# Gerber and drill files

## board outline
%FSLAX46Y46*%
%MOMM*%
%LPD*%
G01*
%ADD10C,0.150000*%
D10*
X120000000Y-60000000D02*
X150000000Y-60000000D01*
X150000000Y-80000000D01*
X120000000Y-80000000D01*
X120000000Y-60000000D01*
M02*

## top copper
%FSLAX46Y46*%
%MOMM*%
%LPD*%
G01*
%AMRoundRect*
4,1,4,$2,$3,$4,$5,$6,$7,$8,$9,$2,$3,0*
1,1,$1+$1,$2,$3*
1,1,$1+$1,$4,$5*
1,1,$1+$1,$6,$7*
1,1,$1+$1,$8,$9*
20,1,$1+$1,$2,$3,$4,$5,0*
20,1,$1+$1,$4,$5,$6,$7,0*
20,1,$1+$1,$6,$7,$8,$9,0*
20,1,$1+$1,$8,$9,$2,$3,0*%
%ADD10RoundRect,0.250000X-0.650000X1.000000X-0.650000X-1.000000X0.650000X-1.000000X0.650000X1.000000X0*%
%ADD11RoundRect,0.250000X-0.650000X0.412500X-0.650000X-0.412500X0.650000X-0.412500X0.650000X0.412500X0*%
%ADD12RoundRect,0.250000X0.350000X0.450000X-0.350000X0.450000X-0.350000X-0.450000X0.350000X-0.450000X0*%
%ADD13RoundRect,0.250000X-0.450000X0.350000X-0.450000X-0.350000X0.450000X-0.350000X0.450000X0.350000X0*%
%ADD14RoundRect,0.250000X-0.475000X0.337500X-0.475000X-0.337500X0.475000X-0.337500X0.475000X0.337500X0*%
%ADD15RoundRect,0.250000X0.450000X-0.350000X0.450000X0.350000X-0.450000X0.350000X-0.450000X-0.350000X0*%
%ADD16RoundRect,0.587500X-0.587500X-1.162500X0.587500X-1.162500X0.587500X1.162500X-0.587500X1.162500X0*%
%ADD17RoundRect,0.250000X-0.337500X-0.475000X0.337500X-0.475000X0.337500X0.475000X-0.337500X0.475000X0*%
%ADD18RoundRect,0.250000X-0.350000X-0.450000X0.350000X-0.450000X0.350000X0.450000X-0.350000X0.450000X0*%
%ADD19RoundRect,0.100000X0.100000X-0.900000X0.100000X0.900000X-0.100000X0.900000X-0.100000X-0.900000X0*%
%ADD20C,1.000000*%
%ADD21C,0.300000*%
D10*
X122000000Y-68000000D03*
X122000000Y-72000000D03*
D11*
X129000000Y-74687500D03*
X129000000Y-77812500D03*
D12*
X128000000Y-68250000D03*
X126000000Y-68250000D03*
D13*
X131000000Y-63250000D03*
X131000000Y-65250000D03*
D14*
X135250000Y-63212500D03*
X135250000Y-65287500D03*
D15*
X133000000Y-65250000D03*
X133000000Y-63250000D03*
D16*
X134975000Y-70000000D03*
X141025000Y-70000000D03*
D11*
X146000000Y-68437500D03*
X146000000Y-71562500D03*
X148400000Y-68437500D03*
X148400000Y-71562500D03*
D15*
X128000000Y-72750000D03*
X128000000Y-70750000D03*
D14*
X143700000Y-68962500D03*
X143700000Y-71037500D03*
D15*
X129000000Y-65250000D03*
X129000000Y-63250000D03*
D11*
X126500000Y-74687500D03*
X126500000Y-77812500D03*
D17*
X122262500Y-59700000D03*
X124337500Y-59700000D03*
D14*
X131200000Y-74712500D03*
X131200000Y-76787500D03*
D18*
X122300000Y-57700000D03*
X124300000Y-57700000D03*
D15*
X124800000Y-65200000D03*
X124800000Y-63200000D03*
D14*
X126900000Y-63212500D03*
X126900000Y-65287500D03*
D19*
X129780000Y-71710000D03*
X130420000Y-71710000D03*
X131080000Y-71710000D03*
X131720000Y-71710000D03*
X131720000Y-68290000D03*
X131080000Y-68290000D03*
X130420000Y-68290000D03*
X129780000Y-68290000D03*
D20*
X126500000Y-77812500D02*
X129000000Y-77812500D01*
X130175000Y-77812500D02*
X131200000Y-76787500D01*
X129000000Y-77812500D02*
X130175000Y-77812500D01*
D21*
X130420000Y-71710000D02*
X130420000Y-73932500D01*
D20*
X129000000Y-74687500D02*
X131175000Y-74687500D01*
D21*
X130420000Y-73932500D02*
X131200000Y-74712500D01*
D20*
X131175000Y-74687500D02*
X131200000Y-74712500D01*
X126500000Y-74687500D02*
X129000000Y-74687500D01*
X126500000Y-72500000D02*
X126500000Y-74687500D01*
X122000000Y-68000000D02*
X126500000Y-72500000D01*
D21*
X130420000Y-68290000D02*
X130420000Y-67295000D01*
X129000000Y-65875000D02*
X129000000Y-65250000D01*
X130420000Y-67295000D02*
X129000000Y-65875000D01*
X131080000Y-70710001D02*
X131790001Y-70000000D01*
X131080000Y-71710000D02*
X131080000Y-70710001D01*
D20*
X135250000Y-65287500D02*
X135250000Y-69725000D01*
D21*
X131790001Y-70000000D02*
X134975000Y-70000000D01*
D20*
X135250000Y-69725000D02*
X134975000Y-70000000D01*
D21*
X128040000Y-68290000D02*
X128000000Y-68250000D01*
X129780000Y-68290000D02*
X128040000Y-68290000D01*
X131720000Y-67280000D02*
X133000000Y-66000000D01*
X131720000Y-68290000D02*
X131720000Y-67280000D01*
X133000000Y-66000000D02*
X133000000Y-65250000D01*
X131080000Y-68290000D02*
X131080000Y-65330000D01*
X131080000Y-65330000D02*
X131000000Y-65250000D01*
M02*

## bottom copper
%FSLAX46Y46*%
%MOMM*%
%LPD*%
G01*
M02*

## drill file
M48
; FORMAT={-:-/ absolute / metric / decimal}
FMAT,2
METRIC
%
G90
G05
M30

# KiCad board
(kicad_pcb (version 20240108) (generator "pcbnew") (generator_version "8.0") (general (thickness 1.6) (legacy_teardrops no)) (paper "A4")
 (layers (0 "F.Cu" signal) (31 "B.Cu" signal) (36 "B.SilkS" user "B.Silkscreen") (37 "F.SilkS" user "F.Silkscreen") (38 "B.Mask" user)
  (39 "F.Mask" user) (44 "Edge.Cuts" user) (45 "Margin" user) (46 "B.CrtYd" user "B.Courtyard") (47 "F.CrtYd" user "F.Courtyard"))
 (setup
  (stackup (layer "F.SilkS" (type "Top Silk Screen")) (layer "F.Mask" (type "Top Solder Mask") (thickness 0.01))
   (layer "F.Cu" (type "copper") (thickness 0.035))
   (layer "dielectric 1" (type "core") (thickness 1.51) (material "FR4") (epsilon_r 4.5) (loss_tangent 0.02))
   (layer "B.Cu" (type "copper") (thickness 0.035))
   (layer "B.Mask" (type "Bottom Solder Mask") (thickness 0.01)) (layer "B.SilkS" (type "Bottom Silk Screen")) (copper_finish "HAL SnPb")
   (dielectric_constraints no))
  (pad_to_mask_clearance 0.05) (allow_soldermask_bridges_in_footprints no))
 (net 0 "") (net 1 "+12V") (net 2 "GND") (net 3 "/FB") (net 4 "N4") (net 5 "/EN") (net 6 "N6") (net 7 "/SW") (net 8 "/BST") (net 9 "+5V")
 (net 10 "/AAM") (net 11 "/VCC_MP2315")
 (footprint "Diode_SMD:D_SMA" (layer "F.Cu") (at 122 70 -90)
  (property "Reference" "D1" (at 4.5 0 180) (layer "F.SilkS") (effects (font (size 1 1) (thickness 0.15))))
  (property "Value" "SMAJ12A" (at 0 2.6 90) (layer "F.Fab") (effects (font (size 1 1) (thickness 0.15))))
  (pad "1" smd roundrect (at -2 0 270) (size 2.5 1.8) (layers "F.Cu" "F.Paste" "F.Mask") (roundrect_rratio 0.1388888889) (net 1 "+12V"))
  (pad "2" smd roundrect (at 2 0 270) (size 2.5 1.8) (layers "F.Cu" "F.Paste" "F.Mask") (roundrect_rratio 0.1388888889) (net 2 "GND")))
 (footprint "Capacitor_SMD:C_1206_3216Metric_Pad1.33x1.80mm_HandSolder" (layer "F.Cu") (at 129 76.25 -90)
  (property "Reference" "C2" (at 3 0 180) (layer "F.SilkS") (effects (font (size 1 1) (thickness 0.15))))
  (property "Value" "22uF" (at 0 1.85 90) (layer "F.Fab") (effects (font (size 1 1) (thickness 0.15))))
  (pad "1" smd roundrect (at -1.5625 0 270) (size 1.325 1.8) (layers "F.Cu" "F.Paste" "F.Mask") (roundrect_rratio 0.188679) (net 1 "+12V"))
  (pad "2" smd roundrect (at 1.5625 0 270) (size 1.325 1.8) (layers "F.Cu" "F.Paste" "F.Mask") (roundrect_rratio 0.188679) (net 2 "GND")))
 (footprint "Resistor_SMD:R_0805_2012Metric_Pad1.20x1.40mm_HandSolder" (layer "F.Cu") (at 127 68.25 180)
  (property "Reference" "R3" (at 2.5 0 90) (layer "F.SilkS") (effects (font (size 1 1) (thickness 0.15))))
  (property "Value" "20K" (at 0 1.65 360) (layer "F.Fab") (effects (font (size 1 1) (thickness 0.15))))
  (pad "1" smd roundrect (at -1 0 180) (size 1.2 1.4) (layers "F.Cu" "F.Paste" "F.Mask") (roundrect_rratio 0.208333) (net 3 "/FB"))
  (pad "2" smd roundrect (at 1 0 180) (size 1.2 1.4) (layers "F.Cu" "F.Paste" "F.Mask") (roundrect_rratio 0.208333) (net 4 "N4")))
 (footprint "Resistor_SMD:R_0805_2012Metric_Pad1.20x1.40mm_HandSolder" (layer "F.Cu") (at 131 64.25 -90)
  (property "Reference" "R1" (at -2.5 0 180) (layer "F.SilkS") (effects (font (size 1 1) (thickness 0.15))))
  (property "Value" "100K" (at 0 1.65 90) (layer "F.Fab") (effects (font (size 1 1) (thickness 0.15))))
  (pad "1" smd roundrect (at -1 0 270) (size 1.2 1.4) (layers "F.Cu" "F.Paste" "F.Mask") (roundrect_rratio 0.208333) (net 1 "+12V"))
  (pad "2" smd roundrect (at 1 0 270) (size 1.2 1.4) (layers "F.Cu" "F.Paste" "F.Mask") (roundrect_rratio 0.208333) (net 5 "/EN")))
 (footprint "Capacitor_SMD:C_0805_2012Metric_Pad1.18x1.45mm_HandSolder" (layer "F.Cu") (at 135.25 64.25 -90)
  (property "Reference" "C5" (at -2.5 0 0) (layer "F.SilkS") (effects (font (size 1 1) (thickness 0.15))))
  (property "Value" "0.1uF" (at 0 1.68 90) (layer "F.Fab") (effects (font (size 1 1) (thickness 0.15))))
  (pad "1" smd roundrect (at -1.0375 0 270) (size 1.175 1.45) (layers "F.Cu" "F.Paste" "F.Mask") (roundrect_rratio 0.212766) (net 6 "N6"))
  (pad "2" smd roundrect (at 1.0375 0 270) (size 1.175 1.45) (layers "F.Cu" "F.Paste" "F.Mask") (roundrect_rratio 0.212766) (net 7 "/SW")))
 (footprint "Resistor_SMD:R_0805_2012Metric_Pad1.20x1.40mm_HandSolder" (layer "F.Cu") (at 133 64.25 90)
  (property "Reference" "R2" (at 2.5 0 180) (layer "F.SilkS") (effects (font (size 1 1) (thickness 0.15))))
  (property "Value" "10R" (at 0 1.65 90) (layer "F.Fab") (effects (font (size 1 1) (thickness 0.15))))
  (pad "1" smd roundrect (at -1 0 90) (size 1.2 1.4) (layers "F.Cu" "F.Paste" "F.Mask") (roundrect_rratio 0.208333) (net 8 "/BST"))
  (pad "2" smd roundrect (at 1 0 90) (size 1.2 1.4) (layers "F.Cu" "F.Paste" "F.Mask") (roundrect_rratio 0.208333) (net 6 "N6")))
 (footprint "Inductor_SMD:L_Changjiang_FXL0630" (layer "F.Cu") (at 138 70)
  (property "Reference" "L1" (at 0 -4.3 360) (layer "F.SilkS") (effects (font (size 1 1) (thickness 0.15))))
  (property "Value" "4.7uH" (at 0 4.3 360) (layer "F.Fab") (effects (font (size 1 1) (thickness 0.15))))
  (pad "1" smd roundrect (at -3.025 0) (size 2.35 3.5) (layers "F.Cu" "F.Paste" "F.Mask") (roundrect_rratio 0.25) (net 7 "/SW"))
  (pad "2" smd roundrect (at 3.025 0) (size 2.35 3.5) (layers "F.Cu" "F.Paste" "F.Mask") (roundrect_rratio 0.25) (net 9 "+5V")))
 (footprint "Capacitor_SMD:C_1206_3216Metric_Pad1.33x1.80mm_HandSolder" (layer "F.Cu") (at 146 70 -90)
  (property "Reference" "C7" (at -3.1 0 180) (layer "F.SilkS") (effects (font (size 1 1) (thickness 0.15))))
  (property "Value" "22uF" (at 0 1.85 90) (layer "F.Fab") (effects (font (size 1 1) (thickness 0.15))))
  (pad "1" smd roundrect (at -1.5625 0 270) (size 1.325 1.8) (layers "F.Cu" "F.Paste" "F.Mask") (roundrect_rratio 0.188679) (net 9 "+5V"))
  (pad "2" smd roundrect (at 1.5625 0 270) (size 1.325 1.8) (layers "F.Cu" "F.Paste" "F.Mask") (roundrect_rratio 0.188679) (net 2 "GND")))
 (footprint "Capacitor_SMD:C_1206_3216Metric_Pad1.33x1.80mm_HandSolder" (layer "F.Cu") (at 148.4 70 -90)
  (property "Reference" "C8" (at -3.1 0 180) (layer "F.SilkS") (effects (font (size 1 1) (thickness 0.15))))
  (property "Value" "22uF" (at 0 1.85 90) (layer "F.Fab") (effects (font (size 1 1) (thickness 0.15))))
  (pad "1" smd roundrect (at -1.5625 0 270) (size 1.325 1.8) (layers "F.Cu" "F.Paste" "F.Mask") (roundrect_rratio 0.188679) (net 9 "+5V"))
  (pad "2" smd roundrect (at 1.5625 0 270) (size 1.325 1.8) (layers "F.Cu" "F.Paste" "F.Mask") (roundrect_rratio 0.188679) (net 2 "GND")))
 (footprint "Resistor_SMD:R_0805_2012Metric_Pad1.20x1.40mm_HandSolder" (layer "F.Cu") (at 128 71.75 90)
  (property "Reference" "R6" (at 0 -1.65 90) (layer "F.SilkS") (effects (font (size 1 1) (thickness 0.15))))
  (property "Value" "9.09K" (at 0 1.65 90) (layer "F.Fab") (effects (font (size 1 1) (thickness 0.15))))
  (pad "1" smd roundrect (at -1 0 90) (size 1.2 1.4) (layers "F.Cu" "F.Paste" "F.Mask") (roundrect_rratio 0.208333) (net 2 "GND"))
  (pad "2" smd roundrect (at 1 0 90) (size 1.2 1.4) (layers "F.Cu" "F.Paste" "F.Mask") (roundrect_rratio 0.208333) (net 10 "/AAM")))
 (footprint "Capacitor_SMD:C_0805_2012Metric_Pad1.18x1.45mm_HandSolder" (layer "F.Cu") (at 143.7 70 -90)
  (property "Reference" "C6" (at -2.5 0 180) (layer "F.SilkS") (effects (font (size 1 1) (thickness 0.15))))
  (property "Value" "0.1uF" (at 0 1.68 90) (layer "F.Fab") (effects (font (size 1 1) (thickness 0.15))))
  (pad "1" smd roundrect (at -1.0375 0 270) (size 1.175 1.45) (layers "F.Cu" "F.Paste" "F.Mask") (roundrect_rratio 0.212766) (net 9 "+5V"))
  (pad "2" smd roundrect (at 1.0375 0 270) (size 1.175 1.45) (layers "F.Cu" "F.Paste" "F.Mask") (roundrect_rratio 0.212766) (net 2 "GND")))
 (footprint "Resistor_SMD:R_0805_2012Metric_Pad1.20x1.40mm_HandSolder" (layer "F.Cu") (at 129 64.25 90)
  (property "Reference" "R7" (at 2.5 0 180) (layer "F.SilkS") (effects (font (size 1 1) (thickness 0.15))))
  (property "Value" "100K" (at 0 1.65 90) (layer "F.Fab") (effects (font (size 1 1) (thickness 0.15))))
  (pad "1" smd roundrect (at -1 0 90) (size 1.2 1.4) (layers "F.Cu" "F.Paste" "F.Mask") (roundrect_rratio 0.208333) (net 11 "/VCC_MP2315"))
  (pad "2" smd roundrect (at 1 0 90) (size 1.2 1.4) (layers "F.Cu" "F.Paste" "F.Mask") (roundrect_rratio 0.208333) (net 10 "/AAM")))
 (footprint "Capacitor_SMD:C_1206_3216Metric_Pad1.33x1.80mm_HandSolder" (layer "F.Cu") (at 126.5 76.25 -90)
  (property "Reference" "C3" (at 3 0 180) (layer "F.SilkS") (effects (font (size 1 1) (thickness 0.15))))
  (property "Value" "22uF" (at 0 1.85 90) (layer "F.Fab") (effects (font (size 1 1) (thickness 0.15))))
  (pad "1" smd roundrect (at -1.5625 0 270) (size 1.325 1.8) (layers "F.Cu" "F.Paste" "F.Mask") (roundrect_rratio 0.188679) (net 1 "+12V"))
  (pad "2" smd roundrect (at 1.5625 0 270) (size 1.325 1.8) (layers "F.Cu" "F.Paste" "F.Mask") (roundrect_rratio 0.188679) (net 2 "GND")))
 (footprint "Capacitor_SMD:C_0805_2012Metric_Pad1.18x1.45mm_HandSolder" (layer "F.Cu") (at 123.3 59.7)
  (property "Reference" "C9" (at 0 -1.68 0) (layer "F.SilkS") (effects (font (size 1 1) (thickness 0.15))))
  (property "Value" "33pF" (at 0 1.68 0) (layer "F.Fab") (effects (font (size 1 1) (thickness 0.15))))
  (pad "1" smd roundrect (at -1.0375 0) (size 1.175 1.45) (layers "F.Cu" "F.Paste" "F.Mask") (roundrect_rratio 0.212766) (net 4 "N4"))
  (pad "2" smd roundrect (at 1.0375 0) (size 1.175 1.45) (layers "F.Cu" "F.Paste" "F.Mask") (roundrect_rratio 0.212766) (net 9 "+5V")))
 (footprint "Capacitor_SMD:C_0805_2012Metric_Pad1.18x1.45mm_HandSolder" (layer "F.Cu") (at 131.2 75.75 -90)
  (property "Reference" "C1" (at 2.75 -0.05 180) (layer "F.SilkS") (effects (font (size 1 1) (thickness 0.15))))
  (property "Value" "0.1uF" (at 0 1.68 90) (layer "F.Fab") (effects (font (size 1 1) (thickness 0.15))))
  (pad "1" smd roundrect (at -1.0375 0 270) (size 1.175 1.45) (layers "F.Cu" "F.Paste" "F.Mask") (roundrect_rratio 0.212766) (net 1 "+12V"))
  (pad "2" smd roundrect (at 1.0375 0 270) (size 1.175 1.45) (layers "F.Cu" "F.Paste" "F.Mask") (roundrect_rratio 0.212766) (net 2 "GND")))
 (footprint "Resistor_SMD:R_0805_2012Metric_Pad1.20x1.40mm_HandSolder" (layer "F.Cu") (at 123.3 57.7)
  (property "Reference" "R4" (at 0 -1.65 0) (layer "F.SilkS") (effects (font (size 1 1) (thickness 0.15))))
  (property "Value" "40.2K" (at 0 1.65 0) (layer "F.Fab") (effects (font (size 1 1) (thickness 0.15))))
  (pad "1" smd roundrect (at -1 0) (size 1.2 1.4) (layers "F.Cu" "F.Paste" "F.Mask") (roundrect_rratio 0.208333) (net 4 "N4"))
  (pad "2" smd roundrect (at 1 0) (size 1.2 1.4) (layers "F.Cu" "F.Paste" "F.Mask") (roundrect_rratio 0.208333) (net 9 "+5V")))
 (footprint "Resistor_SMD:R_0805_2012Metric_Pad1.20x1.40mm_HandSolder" (layer "F.Cu") (at 124.8 64.2 90)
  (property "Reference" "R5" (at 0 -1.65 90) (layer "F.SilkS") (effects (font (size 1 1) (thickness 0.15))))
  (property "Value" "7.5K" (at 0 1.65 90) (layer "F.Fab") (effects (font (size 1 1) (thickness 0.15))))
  (pad "1" smd roundrect (at -1 0 90) (size 1.2 1.4) (layers "F.Cu" "F.Paste" "F.Mask") (roundrect_rratio 0.208333) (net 4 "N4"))
  (pad "2" smd roundrect (at 1 0 90) (size 1.2 1.4) (layers "F.Cu" "F.Paste" "F.Mask") (roundrect_rratio 0.208333) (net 2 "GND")))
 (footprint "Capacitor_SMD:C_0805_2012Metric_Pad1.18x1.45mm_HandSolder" (layer "F.Cu") (at 126.9 64.25 -90)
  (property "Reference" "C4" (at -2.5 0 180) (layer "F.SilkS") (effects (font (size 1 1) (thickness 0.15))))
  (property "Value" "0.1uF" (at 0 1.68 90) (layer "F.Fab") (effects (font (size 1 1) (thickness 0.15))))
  (pad "1" smd roundrect (at -1.0375 0 270) (size 1.175 1.45) (layers "F.Cu" "F.Paste" "F.Mask") (roundrect_rratio 0.212766) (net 2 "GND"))
  (pad "2" smd roundrect (at 1.0375 0 270) (size 1.175 1.45) (layers "F.Cu" "F.Paste" "F.Mask") (roundrect_rratio 0.212766)
   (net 11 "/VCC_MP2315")))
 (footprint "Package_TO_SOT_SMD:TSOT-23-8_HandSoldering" (layer "F.Cu") (at 130.75 70 90)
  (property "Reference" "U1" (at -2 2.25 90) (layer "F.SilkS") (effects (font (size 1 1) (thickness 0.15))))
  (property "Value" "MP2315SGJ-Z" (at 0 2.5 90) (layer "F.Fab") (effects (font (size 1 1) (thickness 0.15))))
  (pad "1" smd roundrect (at -1.71 -0.97 90) (size 2 0.4) (layers "F.Cu" "F.Paste" "F.Mask") (roundrect_rratio 0.25) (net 10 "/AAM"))
  (pad "2" smd roundrect (at -1.71 -0.33 90) (size 2 0.4) (layers "F.Cu" "F.Paste" "F.Mask") (roundrect_rratio 0.25) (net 1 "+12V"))
  (pad "3" smd roundrect (at -1.71 0.33 90) (size 2 0.4) (layers "F.Cu" "F.Paste" "F.Mask") (roundrect_rratio 0.25) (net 7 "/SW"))
  (pad "4" smd roundrect (at -1.71 0.97 90) (size 2 0.4) (layers "F.Cu" "F.Paste" "F.Mask") (roundrect_rratio 0.25) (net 2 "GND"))
  (pad "5" smd roundrect (at 1.71 0.97 90) (size 2 0.4) (layers "F.Cu" "F.Paste" "F.Mask") (roundrect_rratio 0.25) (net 8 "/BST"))
  (pad "6" smd roundrect (at 1.71 0.33 90) (size 2 0.4) (layers "F.Cu" "F.Paste" "F.Mask") (roundrect_rratio 0.25) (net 5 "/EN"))
  (pad "7" smd roundrect (at 1.71 -0.33 90) (size 2 0.4) (layers "F.Cu" "F.Paste" "F.Mask") (roundrect_rratio 0.25) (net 11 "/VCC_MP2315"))
  (pad "8" smd roundrect (at 1.71 -0.97 90) (size 2 0.4) (layers "F.Cu" "F.Paste" "F.Mask") (roundrect_rratio 0.25) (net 3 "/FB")))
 (gr_rect (start 120 60) (end 150 80) (stroke (width 0.15) (type default)) (fill none) (layer "Edge.Cuts"))
 (segment (start 126.5 77.8125) (end 129 77.8125) (width 1) (layer "F.Cu") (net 2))
 (segment (start 130.175 77.8125) (end 131.2 76.7875) (width 1) (layer "F.Cu") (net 2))
 (segment (start 129 77.8125) (end 130.175 77.8125) (width 1) (layer "F.Cu") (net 2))
 (segment (start 130.42 71.71) (end 130.42 73.9325) (width 0.3) (layer "F.Cu") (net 1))
 (segment (start 129 74.6875) (end 131.175 74.6875) (width 1) (layer "F.Cu") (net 1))
 (segment (start 130.42 73.9325) (end 131.2 74.7125) (width 0.3) (layer "F.Cu") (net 1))
 (segment (start 131.175 74.6875) (end 131.2 74.7125) (width 1) (layer "F.Cu") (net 1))
 (segment (start 126.5 74.6875) (end 129 74.6875) (width 1) (layer "F.Cu") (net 1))
 (segment (start 126.5 72.5) (end 126.5 74.6875) (width 1) (layer "F.Cu") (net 1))
 (segment (start 122 68) (end 126.5 72.5) (width 1) (layer "F.Cu") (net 1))
 (segment (start 130.42 68.29) (end 130.42 67.295) (width 0.3) (layer "F.Cu") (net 11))
 (segment (start 129 65.875) (end 129 65.25) (width 0.3) (layer "F.Cu") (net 11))
 (segment (start 130.42 67.295) (end 129 65.875) (width 0.3) (layer "F.Cu") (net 11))
 (segment (start 131.08 70.710001) (end 131.790001 70) (width 0.3) (layer "F.Cu") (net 7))
 (segment (start 131.08 71.71) (end 131.08 70.710001) (width 0.3) (layer "F.Cu") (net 7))
 (segment (start 135.25 65.2875) (end 135.25 69.725) (width 1) (layer "F.Cu") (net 7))
 (segment (start 131.790001 70) (end 134.975 70) (width 0.3) (layer "F.Cu") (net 7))
 (segment (start 135.25 69.725) (end 134.975 70) (width 1) (layer "F.Cu") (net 7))
 (segment (start 128.04 68.29) (end 128 68.25) (width 0.3) (layer "F.Cu") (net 3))
 (segment (start 129.78 68.29) (end 128.04 68.29) (width 0.3) (layer "F.Cu") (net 3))
 (segment (start 131.72 67.28) (end 133 66) (width 0.3) (layer "F.Cu") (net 8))
 (segment (start 131.72 68.29) (end 131.72 67.28) (width 0.3) (layer "F.Cu") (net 8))
 (segment (start 133 66) (end 133 65.25) (width 0.3) (layer "F.Cu") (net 8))
 (segment (start 131.08 68.29) (end 131.08 65.33) (width 0.3) (layer "F.Cu") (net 5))
 (segment (start 131.08 65.33) (end 131 65.25) (width 0.3) (layer "F.Cu") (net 5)))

